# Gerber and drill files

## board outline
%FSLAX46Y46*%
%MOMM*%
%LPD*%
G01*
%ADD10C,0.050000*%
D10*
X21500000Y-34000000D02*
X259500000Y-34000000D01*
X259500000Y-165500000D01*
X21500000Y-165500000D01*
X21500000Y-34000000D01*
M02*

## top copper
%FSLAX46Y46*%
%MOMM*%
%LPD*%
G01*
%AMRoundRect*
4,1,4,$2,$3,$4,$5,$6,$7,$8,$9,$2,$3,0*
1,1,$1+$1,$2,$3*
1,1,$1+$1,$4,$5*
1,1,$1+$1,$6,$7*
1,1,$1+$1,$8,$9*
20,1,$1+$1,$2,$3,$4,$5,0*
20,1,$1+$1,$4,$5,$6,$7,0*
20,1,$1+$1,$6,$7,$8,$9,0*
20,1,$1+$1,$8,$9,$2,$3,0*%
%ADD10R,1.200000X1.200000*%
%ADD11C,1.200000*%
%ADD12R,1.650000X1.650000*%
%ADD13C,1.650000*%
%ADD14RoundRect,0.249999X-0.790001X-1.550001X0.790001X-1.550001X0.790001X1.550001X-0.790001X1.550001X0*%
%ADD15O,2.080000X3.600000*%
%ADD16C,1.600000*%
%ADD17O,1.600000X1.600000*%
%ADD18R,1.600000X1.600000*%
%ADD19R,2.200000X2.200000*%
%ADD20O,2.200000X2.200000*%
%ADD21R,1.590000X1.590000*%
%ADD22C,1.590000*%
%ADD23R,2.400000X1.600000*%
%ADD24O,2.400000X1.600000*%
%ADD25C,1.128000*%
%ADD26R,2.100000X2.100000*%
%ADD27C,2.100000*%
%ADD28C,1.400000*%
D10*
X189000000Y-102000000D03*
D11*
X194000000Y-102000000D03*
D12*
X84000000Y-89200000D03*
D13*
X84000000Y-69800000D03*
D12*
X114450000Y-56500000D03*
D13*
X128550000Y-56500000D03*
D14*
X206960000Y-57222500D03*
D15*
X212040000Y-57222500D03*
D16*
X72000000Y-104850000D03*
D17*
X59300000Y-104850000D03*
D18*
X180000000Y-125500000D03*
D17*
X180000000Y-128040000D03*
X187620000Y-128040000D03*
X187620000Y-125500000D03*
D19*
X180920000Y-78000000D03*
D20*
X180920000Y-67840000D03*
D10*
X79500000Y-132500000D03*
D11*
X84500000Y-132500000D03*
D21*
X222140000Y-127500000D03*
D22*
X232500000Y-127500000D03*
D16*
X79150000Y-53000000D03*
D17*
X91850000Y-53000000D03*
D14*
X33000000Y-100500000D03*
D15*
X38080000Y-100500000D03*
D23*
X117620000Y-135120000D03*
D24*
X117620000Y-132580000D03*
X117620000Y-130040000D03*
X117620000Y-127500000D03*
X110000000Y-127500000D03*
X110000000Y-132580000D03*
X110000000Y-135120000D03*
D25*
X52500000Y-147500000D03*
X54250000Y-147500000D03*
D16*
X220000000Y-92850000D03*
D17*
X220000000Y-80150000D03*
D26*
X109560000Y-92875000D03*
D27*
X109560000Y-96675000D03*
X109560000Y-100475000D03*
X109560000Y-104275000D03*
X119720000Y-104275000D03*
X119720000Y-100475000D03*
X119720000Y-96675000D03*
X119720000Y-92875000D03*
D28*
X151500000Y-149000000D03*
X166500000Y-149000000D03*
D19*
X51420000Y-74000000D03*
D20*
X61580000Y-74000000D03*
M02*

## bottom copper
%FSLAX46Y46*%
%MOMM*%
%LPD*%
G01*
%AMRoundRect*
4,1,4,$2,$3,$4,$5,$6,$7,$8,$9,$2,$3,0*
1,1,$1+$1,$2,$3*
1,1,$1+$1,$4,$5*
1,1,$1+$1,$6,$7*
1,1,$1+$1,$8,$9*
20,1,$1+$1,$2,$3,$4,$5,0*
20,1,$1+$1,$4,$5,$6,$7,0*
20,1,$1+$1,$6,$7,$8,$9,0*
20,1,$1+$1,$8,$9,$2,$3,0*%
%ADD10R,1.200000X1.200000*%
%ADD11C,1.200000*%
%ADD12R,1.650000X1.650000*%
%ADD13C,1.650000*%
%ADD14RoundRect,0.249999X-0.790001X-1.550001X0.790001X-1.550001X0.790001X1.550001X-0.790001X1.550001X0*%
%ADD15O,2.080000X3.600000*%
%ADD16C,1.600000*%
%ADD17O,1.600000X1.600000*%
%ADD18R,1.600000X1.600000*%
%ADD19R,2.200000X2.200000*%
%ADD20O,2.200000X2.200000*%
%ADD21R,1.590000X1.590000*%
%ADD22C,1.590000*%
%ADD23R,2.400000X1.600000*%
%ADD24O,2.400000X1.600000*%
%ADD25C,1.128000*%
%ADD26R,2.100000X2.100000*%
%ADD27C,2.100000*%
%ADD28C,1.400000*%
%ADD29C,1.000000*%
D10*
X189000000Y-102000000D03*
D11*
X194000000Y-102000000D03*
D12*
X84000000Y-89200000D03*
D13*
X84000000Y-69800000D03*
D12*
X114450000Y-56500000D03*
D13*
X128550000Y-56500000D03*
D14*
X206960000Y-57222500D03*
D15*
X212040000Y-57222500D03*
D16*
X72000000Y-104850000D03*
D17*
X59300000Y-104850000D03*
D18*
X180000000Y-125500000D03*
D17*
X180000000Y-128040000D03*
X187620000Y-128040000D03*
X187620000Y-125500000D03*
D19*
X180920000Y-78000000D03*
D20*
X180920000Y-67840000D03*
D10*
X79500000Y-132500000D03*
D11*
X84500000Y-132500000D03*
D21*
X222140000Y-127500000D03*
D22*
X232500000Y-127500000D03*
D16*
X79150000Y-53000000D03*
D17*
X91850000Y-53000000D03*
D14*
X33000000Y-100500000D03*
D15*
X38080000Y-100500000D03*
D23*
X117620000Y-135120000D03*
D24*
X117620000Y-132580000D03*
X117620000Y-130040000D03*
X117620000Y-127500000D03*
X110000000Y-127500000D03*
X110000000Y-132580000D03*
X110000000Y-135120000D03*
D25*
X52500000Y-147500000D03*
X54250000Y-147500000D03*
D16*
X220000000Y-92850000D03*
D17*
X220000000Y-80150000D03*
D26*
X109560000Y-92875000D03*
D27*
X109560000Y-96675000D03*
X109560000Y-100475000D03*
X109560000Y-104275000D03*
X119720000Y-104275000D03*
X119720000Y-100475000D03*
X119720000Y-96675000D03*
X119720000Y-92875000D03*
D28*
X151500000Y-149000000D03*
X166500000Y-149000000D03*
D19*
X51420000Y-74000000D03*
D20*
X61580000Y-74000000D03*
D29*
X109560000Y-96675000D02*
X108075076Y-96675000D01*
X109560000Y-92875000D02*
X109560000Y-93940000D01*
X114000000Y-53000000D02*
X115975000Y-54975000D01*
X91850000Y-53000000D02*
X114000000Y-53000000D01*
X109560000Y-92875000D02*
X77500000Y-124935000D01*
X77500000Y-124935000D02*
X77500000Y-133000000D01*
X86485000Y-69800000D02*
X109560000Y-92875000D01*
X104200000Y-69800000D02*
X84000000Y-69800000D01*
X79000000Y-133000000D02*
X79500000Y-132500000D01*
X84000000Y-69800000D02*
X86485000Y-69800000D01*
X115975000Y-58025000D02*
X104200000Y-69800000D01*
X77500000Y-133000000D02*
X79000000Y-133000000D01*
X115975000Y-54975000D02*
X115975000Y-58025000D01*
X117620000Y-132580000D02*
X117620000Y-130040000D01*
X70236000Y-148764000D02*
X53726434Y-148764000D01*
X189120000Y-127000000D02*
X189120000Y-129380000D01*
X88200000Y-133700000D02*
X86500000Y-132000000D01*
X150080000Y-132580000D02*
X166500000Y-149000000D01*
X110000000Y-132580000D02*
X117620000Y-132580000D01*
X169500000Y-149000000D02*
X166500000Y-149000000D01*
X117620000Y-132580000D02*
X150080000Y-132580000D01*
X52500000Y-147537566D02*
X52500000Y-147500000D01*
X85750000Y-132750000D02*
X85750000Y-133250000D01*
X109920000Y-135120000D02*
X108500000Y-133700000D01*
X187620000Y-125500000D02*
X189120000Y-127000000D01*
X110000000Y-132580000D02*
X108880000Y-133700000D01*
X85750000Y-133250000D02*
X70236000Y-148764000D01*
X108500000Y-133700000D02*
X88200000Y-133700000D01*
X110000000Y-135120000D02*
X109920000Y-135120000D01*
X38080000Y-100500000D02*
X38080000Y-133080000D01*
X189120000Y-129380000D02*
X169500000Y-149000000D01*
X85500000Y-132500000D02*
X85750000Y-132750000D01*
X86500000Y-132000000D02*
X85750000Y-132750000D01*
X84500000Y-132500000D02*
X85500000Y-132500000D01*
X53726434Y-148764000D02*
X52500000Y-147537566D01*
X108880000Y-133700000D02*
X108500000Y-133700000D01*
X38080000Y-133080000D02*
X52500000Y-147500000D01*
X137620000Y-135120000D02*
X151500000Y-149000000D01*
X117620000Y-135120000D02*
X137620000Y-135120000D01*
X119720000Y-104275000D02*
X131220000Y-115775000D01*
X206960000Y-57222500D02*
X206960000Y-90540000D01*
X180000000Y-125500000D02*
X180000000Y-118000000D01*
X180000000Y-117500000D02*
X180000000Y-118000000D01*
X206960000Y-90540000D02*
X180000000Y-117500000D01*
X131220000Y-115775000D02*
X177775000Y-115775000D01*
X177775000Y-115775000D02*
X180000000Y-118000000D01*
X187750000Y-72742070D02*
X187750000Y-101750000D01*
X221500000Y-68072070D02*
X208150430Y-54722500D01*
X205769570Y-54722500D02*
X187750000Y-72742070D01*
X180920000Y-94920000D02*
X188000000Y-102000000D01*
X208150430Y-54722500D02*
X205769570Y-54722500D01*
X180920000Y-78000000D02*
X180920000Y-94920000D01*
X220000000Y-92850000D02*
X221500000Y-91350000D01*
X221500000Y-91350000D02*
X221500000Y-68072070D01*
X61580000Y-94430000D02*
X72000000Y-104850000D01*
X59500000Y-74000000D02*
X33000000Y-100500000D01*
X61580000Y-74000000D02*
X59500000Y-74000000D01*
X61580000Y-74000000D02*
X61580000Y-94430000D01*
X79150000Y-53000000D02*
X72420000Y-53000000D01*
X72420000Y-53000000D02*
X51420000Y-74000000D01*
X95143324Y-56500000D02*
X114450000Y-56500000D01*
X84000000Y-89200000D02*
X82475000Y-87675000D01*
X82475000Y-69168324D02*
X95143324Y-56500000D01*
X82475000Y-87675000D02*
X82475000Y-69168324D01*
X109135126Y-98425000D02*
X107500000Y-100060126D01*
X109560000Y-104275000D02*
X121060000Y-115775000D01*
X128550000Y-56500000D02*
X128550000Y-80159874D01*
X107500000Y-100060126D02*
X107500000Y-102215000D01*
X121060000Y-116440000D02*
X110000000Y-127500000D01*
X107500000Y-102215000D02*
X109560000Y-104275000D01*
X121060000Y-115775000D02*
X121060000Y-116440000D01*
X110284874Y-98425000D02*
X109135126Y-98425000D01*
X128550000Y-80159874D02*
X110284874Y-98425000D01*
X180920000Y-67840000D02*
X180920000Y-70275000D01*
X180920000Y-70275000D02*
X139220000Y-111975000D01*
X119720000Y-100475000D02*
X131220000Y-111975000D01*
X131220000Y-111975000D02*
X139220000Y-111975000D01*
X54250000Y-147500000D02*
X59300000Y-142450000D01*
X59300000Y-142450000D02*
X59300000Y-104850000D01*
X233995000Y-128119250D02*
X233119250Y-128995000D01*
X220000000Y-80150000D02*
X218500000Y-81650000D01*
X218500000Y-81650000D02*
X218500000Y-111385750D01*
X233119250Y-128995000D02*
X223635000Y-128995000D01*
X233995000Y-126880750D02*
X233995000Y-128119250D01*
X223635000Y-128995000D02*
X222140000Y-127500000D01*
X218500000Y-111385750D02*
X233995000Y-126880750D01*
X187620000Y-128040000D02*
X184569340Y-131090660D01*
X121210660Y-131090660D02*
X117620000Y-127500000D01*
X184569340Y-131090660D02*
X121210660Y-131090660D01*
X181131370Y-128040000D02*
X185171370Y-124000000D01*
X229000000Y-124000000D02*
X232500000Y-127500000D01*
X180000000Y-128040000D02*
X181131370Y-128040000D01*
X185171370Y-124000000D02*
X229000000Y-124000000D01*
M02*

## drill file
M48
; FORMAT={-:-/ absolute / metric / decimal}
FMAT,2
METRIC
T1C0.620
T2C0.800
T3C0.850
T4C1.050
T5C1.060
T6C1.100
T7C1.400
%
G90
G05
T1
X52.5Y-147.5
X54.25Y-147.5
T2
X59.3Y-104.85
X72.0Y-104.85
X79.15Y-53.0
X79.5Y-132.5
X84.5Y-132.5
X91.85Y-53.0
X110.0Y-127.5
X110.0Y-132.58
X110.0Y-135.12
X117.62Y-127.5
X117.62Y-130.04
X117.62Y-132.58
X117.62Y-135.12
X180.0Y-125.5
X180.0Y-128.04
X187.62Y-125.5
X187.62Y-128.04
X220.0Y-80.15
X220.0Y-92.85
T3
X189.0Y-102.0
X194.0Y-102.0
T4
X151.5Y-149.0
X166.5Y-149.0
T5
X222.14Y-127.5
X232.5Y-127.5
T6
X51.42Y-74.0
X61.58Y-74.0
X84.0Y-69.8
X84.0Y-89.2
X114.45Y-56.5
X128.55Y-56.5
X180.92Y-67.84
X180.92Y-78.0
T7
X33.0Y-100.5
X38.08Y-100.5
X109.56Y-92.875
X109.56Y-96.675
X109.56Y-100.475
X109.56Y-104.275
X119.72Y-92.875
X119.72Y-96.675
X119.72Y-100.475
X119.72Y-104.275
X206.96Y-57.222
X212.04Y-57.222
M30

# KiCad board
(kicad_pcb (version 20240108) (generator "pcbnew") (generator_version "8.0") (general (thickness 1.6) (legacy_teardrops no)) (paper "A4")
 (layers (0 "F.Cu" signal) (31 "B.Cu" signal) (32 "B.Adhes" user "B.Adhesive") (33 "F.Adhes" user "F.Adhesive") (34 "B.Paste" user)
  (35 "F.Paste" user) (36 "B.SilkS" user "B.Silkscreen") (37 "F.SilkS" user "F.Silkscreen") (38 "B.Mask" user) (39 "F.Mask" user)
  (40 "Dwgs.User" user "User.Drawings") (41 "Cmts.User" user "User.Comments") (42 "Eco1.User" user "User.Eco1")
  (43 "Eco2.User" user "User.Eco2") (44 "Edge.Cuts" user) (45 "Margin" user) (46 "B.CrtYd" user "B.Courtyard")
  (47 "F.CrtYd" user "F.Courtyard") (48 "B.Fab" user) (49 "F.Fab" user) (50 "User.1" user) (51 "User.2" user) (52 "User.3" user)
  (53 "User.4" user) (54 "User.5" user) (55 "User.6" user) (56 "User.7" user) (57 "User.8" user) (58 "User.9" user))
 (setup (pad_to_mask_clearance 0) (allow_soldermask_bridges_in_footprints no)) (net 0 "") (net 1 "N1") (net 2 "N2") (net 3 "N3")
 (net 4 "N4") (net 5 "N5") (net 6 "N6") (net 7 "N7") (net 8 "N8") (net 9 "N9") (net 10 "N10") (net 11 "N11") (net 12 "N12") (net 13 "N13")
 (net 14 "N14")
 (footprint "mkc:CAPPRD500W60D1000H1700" (layer "F.Cu") (at 191.5 102)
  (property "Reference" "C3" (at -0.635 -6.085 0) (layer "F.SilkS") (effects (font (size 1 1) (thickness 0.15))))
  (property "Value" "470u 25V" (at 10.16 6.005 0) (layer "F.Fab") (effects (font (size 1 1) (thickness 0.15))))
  (pad "1" thru_hole rect (at -2.5 0) (size 1.2 1.2) (drill 0.85) (layers "*.Cu" "*.Mask") (remove_unused_layers no) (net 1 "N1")
   (solder_mask_margin 0.102))
  (pad "2" thru_hole circle (at 2.5 0) (size 1.2 1.2) (drill 0.85) (layers "*.Cu" "*.Mask") (remove_unused_layers no) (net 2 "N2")
   (solder_mask_margin 0.102)))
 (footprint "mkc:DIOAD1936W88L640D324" (layer "F.Cu") (at 84 89.2 90)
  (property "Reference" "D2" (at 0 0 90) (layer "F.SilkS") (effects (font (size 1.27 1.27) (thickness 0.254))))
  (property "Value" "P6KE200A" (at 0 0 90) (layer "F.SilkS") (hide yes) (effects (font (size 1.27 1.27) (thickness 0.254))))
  (pad "1" thru_hole rect (at 0 0 90) (size 1.65 1.65) (drill 1.1) (layers "*.Cu" "*.Mask") (remove_unused_layers no) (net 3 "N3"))
  (pad "2" thru_hole circle (at 19.4 0 90) (size 1.65 1.65) (drill 1.1) (layers "*.Cu" "*.Mask") (remove_unused_layers no) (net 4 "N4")))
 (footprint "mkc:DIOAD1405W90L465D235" (layer "F.Cu") (at 114.45 56.5)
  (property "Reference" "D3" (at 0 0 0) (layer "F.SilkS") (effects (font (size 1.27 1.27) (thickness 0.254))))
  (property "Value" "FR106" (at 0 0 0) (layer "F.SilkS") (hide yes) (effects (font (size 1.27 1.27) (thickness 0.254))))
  (pad "1" thru_hole rect (at 0 0) (size 1.65 1.65) (drill 1.1) (layers "*.Cu" "*.Mask") (remove_unused_layers no) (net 3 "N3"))
  (pad "2" thru_hole circle (at 14.1 0) (size 1.65 1.65) (drill 1.1) (layers "*.Cu" "*.Mask") (remove_unused_layers no) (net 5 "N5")))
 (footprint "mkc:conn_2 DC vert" (layer "F.Cu") (at 206.96 57.2225)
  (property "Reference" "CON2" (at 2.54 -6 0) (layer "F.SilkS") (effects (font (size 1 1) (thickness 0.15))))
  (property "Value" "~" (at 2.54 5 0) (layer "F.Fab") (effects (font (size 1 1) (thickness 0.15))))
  (pad "1" thru_hole roundrect (at 0 0) (size 2.08 3.6) (drill 1.4) (layers "*.Cu" "*.Mask") (remove_unused_layers no)
   (roundrect_rratio 0.120192) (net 2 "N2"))
  (pad "2" thru_hole oval (at 5.08 0) (size 2.08 3.6) (drill 1.4) (layers "*.Cu" "*.Mask") (remove_unused_layers no) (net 1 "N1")))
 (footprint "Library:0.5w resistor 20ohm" (layer "F.Cu") (at 72 104.85 180)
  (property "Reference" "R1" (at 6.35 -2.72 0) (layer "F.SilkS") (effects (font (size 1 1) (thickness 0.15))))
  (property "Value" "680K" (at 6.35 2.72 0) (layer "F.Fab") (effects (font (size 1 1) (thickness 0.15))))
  (pad "1" thru_hole circle (at 0 0 180) (size 1.6 1.6) (drill 0.8) (layers "*.Cu" "*.Mask") (remove_unused_layers no) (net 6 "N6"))
  (pad "2" thru_hole oval (at 12.7 0 180) (size 1.6 1.6) (drill 0.8) (layers "*.Cu" "*.Mask") (remove_unused_layers no) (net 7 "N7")))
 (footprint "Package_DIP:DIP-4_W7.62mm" (layer "F.Cu") (at 180 125.5)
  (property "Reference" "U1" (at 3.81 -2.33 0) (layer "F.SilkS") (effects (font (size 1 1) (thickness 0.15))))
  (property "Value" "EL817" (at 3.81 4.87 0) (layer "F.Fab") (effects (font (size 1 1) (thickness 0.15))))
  (pad "1" thru_hole rect (at 0 0) (size 1.6 1.6) (drill 0.8) (layers "*.Cu" "*.Mask") (remove_unused_layers no) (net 2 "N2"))
  (pad "2" thru_hole oval (at 0 2.54) (size 1.6 1.6) (drill 0.8) (layers "*.Cu" "*.Mask") (remove_unused_layers no) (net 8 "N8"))
  (pad "3" thru_hole oval (at 7.62 2.54) (size 1.6 1.6) (drill 0.8) (layers "*.Cu" "*.Mask") (remove_unused_layers no) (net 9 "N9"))
  (pad "4" thru_hole oval (at 7.62 0) (size 1.6 1.6) (drill 0.8) (layers "*.Cu" "*.Mask") (remove_unused_layers no) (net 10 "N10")))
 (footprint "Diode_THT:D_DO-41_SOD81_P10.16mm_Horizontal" (layer "F.Cu") (at 180.92 78 90)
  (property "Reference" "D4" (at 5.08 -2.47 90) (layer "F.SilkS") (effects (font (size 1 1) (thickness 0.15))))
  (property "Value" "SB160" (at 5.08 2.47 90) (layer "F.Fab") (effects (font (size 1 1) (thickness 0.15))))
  (pad "1" thru_hole rect (at 0 0 90) (size 2.2 2.2) (drill 1.1) (layers "*.Cu" "*.Mask") (remove_unused_layers no) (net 1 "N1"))
  (pad "2" thru_hole oval (at 10.16 0 90) (size 2.2 2.2) (drill 1.1) (layers "*.Cu" "*.Mask") (remove_unused_layers no) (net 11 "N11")))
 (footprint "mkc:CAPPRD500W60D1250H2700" (layer "F.Cu") (at 82 132.5)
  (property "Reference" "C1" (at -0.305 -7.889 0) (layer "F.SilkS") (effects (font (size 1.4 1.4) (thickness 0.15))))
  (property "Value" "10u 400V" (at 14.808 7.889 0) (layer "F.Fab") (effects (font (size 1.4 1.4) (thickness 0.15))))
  (pad "1" thru_hole rect (at -2.5 0) (size 1.2 1.2) (drill 0.8) (layers "*.Cu" "*.Mask") (remove_unused_layers no) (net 4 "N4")
   (solder_mask_margin 0.102))
  (pad "2" thru_hole circle (at 2.5 0) (size 1.2 1.2) (drill 0.8) (layers "*.Cu" "*.Mask") (remove_unused_layers no) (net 10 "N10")
   (solder_mask_margin 0.102)))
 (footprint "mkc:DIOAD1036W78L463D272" (layer "F.Cu") (at 227.32 127.5)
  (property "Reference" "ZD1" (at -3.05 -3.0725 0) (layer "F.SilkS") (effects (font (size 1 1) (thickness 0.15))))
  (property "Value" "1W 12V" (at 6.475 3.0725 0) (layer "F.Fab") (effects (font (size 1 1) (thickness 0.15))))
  (pad "1" thru_hole rect (at -5.18 0) (size 1.59 1.59) (drill 1.06) (layers "*.Cu" "*.Mask") (remove_unused_layers no) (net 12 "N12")
   (solder_mask_margin 0.102))
  (pad "2" thru_hole circle (at 5.18 0) (size 1.59 1.59) (drill 1.06) (layers "*.Cu" "*.Mask") (remove_unused_layers no) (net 8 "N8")
   (solder_mask_margin 0.102)))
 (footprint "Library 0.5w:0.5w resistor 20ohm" (layer "F.Cu") (at 79.15 53)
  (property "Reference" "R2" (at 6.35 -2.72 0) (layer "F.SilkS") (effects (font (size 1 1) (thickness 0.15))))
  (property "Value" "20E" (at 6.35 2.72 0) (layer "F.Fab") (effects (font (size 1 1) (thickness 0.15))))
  (pad "1" thru_hole circle (at 0 0) (size 1.6 1.6) (drill 0.8) (layers "*.Cu" "*.Mask") (remove_unused_layers no) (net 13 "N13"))
  (pad "2" thru_hole oval (at 12.7 0) (size 1.6 1.6) (drill 0.8) (layers "*.Cu" "*.Mask") (remove_unused_layers no) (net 4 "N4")))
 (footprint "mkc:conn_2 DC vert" (layer "F.Cu") (at 33 100.5)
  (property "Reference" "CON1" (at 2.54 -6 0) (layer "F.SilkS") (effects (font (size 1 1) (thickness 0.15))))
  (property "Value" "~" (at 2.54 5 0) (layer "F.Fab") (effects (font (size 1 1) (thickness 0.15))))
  (pad "1" thru_hole roundrect (at 0 0) (size 2.08 3.6) (drill 1.4) (layers "*.Cu" "*.Mask") (remove_unused_layers no)
   (roundrect_rratio 0.120192) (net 6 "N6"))
  (pad "2" thru_hole oval (at 5.08 0) (size 2.08 3.6) (drill 1.4) (layers "*.Cu" "*.Mask") (remove_unused_layers no) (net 10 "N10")))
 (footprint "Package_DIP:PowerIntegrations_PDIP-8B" (layer "F.Cu") (at 117.62 135.12 180)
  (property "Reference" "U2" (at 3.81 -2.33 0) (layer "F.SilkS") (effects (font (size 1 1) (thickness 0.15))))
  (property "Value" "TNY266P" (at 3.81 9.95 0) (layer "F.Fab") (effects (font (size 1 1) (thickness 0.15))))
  (pad "1" thru_hole rect (at 0 0 180) (size 2.4 1.6) (drill 0.8) (layers "*.Cu" "*.Mask") (remove_unused_layers no) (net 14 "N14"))
  (pad "2" thru_hole oval (at 0 2.54 180) (size 2.4 1.6) (drill 0.8) (layers "*.Cu" "*.Mask") (remove_unused_layers no) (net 10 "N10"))
  (pad "3" thru_hole oval (at 0 5.08 180) (size 2.4 1.6) (drill 0.8) (layers "*.Cu" "*.Mask") (remove_unused_layers no) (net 10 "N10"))
  (pad "4" thru_hole oval (at 0 7.62 180) (size 2.4 1.6) (drill 0.8) (layers "*.Cu" "*.Mask") (remove_unused_layers no) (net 9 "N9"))
  (pad "5" thru_hole oval (at 7.62 7.62 180) (size 2.4 1.6) (drill 0.8) (layers "*.Cu" "*.Mask") (remove_unused_layers no) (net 5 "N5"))
  (pad "7" thru_hole oval (at 7.62 2.54 180) (size 2.4 1.6) (drill 0.8) (layers "*.Cu" "*.Mask") (remove_unused_layers no) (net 10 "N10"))
  (pad "8" thru_hole oval (at 7.62 0 180) (size 2.4 1.6) (drill 0.8) (layers "*.Cu" "*.Mask") (remove_unused_layers no) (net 10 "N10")))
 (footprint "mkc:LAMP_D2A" (layer "F.Cu") (at 53.375 147.5)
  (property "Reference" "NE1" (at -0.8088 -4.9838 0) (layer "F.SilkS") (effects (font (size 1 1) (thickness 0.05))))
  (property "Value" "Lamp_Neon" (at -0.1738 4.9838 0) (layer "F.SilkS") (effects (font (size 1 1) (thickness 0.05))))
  (pad "1" thru_hole circle (at -0.875 0) (size 1.128 1.128) (drill 0.62) (layers "*.Cu" "*.Mask") (remove_unused_layers no) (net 10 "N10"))
  (pad "2" thru_hole circle (at 0.875 0) (size 1.128 1.128) (drill 0.62) (layers "*.Cu" "*.Mask") (remove_unused_layers no) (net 7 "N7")))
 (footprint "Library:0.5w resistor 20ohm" (layer "F.Cu") (at 220 92.85 90)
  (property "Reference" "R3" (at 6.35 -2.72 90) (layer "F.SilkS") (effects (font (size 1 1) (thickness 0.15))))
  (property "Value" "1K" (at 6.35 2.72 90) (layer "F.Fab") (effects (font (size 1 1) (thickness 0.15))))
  (pad "1" thru_hole circle (at 0 0 90) (size 1.6 1.6) (drill 0.8) (layers "*.Cu" "*.Mask") (remove_unused_layers no) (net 1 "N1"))
  (pad "2" thru_hole oval (at 12.7 0 90) (size 1.6 1.6) (drill 0.8) (layers "*.Cu" "*.Mask") (remove_unused_layers no) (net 12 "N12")))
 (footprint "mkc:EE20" (layer "F.Cu") (at 109.56 92.875)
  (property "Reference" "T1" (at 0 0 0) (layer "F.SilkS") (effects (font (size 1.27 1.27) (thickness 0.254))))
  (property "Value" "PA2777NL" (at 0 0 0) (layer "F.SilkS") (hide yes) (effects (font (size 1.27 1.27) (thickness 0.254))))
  (pad "1" thru_hole rect (at 0 0) (size 2.1 2.1) (drill 1.4) (layers "*.Cu" "*.Mask") (remove_unused_layers no) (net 4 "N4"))
  (pad "2" thru_hole circle (at 0 3.8) (size 2.1 2.1) (drill 1.4) (layers "*.Cu" "*.Mask") (remove_unused_layers no))
  (pad "3" thru_hole circle (at 0 7.6) (size 2.1 2.1) (drill 1.4) (layers "*.Cu" "*.Mask") (remove_unused_layers no))
  (pad "4" thru_hole circle (at 0 11.4) (size 2.1 2.1) (drill 1.4) (layers "*.Cu" "*.Mask") (remove_unused_layers no) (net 5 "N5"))
  (pad "7" thru_hole circle (at 10.16 11.4) (size 2.1 2.1) (drill 1.4) (layers "*.Cu" "*.Mask") (remove_unused_layers no) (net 2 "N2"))
  (pad "8" thru_hole circle (at 10.16 7.6) (size 2.1 2.1) (drill 1.4) (layers "*.Cu" "*.Mask") (remove_unused_layers no) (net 11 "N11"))
  (pad "9" thru_hole circle (at 10.16 3.8) (size 2.1 2.1) (drill 1.4) (layers "*.Cu" "*.Mask") (remove_unused_layers no))
  (pad "10" thru_hole circle (at 10.16 0) (size 2.1 2.1) (drill 1.4) (layers "*.Cu" "*.Mask") (remove_unused_layers no)))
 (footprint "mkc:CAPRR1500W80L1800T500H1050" (layer "F.Cu") (at 159 149)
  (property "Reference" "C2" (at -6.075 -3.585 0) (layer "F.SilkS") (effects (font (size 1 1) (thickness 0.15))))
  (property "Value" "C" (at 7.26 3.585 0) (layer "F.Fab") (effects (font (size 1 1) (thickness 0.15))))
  (pad "1" thru_hole circle (at -7.5 0) (size 1.4 1.4) (drill 1.05) (layers "*.Cu" "*.Mask") (remove_unused_layers no) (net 14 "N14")
   (solder_mask_margin 0.102))
  (pad "2" thru_hole circle (at 7.5 0) (size 1.4 1.4) (drill 1.05) (layers "*.Cu" "*.Mask") (remove_unused_layers no) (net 10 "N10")
   (solder_mask_margin 0.102)))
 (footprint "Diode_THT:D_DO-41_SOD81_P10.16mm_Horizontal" (layer "F.Cu") (at 51.42 74)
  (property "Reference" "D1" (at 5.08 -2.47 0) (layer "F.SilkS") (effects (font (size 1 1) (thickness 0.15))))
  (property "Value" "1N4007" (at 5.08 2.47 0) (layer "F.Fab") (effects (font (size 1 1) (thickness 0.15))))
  (pad "1" thru_hole rect (at 0 0) (size 2.2 2.2) (drill 1.1) (layers "*.Cu" "*.Mask") (remove_unused_layers no) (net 13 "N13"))
  (pad "2" thru_hole oval (at 10.16 0) (size 2.2 2.2) (drill 1.1) (layers "*.Cu" "*.Mask") (remove_unused_layers no) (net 6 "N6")))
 (gr_rect (start 21.5 34) (end 259.5 165.5) (stroke (width 0.05) (type default)) (fill none) (layer "Edge.Cuts"))
 (segment (start 109.56 96.675) (end 108.075076 96.675) (width 1) (layer "B.Cu") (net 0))
 (segment (start 109.56 92.875) (end 109.56 93.94) (width 1) (layer "B.Cu") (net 4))
 (segment (start 114 53) (end 115.975 54.975) (width 1) (layer "B.Cu") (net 4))
 (segment (start 91.85 53) (end 114 53) (width 1) (layer "B.Cu") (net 4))
 (segment (start 109.56 92.875) (end 77.5 124.935) (width 1) (layer "B.Cu") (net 4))
 (segment (start 77.5 124.935) (end 77.5 133) (width 1) (layer "B.Cu") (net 4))
 (segment (start 86.485 69.8) (end 109.56 92.875) (width 1) (layer "B.Cu") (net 4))
 (segment (start 104.2 69.8) (end 84 69.8) (width 1) (layer "B.Cu") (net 4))
 (segment (start 79 133) (end 79.5 132.5) (width 1) (layer "B.Cu") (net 4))
 (segment (start 84 69.8) (end 86.485 69.8) (width 1) (layer "B.Cu") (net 4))
 (segment (start 115.975 58.025) (end 104.2 69.8) (width 1) (layer "B.Cu") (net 4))
 (segment (start 77.5 133) (end 79 133) (width 1) (layer "B.Cu") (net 4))
 (segment (start 115.975 54.975) (end 115.975 58.025) (width 1) (layer "B.Cu") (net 4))
 (segment (start 117.62 132.58) (end 117.62 130.04) (width 1) (layer "B.Cu") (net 10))
 (segment (start 70.236 148.764) (end 53.726434 148.764) (width 1) (layer "B.Cu") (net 10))
 (segment (start 189.12 127) (end 189.12 129.38) (width 1) (layer "B.Cu") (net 10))
 (segment (start 88.2 133.7) (end 86.5 132) (width 1) (layer "B.Cu") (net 10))
 (segment (start 150.08 132.58) (end 166.5 149) (width 1) (layer "B.Cu") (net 10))
 (segment (start 110 132.58) (end 117.62 132.58) (width 1) (layer "B.Cu") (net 10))
 (segment (start 169.5 149) (end 166.5 149) (width 1) (layer "B.Cu") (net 10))
 (segment (start 117.62 132.58) (end 150.08 132.58) (width 1) (layer "B.Cu") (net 10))
 (segment (start 52.5 147.537566) (end 52.5 147.5) (width 1) (layer "B.Cu") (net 10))
 (segment (start 85.75 132.75) (end 85.75 133.25) (width 1) (layer "B.Cu") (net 10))
 (segment (start 109.92 135.12) (end 108.5 133.7) (width 1) (layer "B.Cu") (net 10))
 (segment (start 187.62 125.5) (end 189.12 127) (width 1) (layer "B.Cu") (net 10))
 (segment (start 110 132.58) (end 108.88 133.7) (width 1) (layer "B.Cu") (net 10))
 (segment (start 85.75 133.25) (end 70.236 148.764) (width 1) (layer "B.Cu") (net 10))
 (segment (start 108.5 133.7) (end 88.2 133.7) (width 1) (layer "B.Cu") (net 10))
 (segment (start 110 135.12) (end 109.92 135.12) (width 1) (layer "B.Cu") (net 10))
 (segment (start 38.08 100.5) (end 38.08 133.08) (width 1) (layer "B.Cu") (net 10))
 (segment (start 189.12 129.38) (end 169.5 149) (width 1) (layer "B.Cu") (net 10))
 (segment (start 85.5 132.5) (end 85.75 132.75) (width 1) (layer "B.Cu") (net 10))
 (segment (start 86.5 132) (end 85.75 132.75) (width 1) (layer "B.Cu") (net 10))
 (segment (start 84.5 132.5) (end 85.5 132.5) (width 1) (layer "B.Cu") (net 10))
 (segment (start 53.726434 148.764) (end 52.5 147.537566) (width 1) (layer "B.Cu") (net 10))
 (segment (start 108.88 133.7) (end 108.5 133.7) (width 1) (layer "B.Cu") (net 10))
 (segment (start 38.08 133.08) (end 52.5 147.5) (width 1) (layer "B.Cu") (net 10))
 (segment (start 137.62 135.12) (end 151.5 149) (width 1) (layer "B.Cu") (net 14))
 (segment (start 117.62 135.12) (end 137.62 135.12) (width 1) (layer "B.Cu") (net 14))
 (segment (start 119.72 104.275) (end 131.22 115.775) (width 1) (layer "B.Cu") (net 2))
 (segment (start 206.96 57.2225) (end 206.96 90.54) (width 1) (layer "B.Cu") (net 2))
 (segment (start 180 125.5) (end 180 118) (width 1) (layer "B.Cu") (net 2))
 (segment (start 180 117.5) (end 180 118) (width 1) (layer "B.Cu") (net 2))
 (segment (start 206.96 90.54) (end 180 117.5) (width 1) (layer "B.Cu") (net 2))
 (segment (start 131.22 115.775) (end 177.775 115.775) (width 1) (layer "B.Cu") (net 2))
 (segment (start 177.775 115.775) (end 180 118) (width 1) (layer "B.Cu") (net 2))
 (segment (start 187.75 72.74207) (end 187.75 101.75) (width 1) (layer "B.Cu") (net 1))
 (segment (start 221.5 68.07207) (end 208.15043 54.7225) (width 1) (layer "B.Cu") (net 1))
 (segment (start 205.76957 54.7225) (end 187.75 72.74207) (width 1) (layer "B.Cu") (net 1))
 (segment (start 180.92 94.92) (end 188 102) (width 1) (layer "B.Cu") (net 1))
 (segment (start 208.15043 54.7225) (end 205.76957 54.7225) (width 1) (layer "B.Cu") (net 1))
 (segment (start 180.92 78) (end 180.92 94.92) (width 1) (layer "B.Cu") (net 1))
 (segment (start 220 92.85) (end 221.5 91.35) (width 1) (layer "B.Cu") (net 1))
 (segment (start 221.5 91.35) (end 221.5 68.07207) (width 1) (layer "B.Cu") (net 1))
 (segment (start 61.58 94.43) (end 72 104.85) (width 1) (layer "B.Cu") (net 6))
 (segment (start 59.5 74) (end 33 100.5) (width 1) (layer "B.Cu") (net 6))
 (segment (start 61.58 74) (end 59.5 74) (width 1) (layer "B.Cu") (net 6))
 (segment (start 61.58 74) (end 61.58 94.43) (width 1) (layer "B.Cu") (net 6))
 (segment (start 79.15 53) (end 72.42 53) (width 1) (layer "B.Cu") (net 13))
 (segment (start 72.42 53) (end 51.42 74) (width 1) (layer "B.Cu") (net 13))
 (segment (start 95.143324 56.5) (end 114.45 56.5) (width 1) (layer "B.Cu") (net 3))
 (segment (start 84 89.2) (end 82.475 87.675) (width 1) (layer "B.Cu") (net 3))
 (segment (start 82.475 69.168324) (end 95.143324 56.5) (width 1) (layer "B.Cu") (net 3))
 (segment (start 82.475 87.675) (end 82.475 69.168324) (width 1) (layer "B.Cu") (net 3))
 (segment (start 109.135126 98.425) (end 107.5 100.060126) (width 1) (layer "B.Cu") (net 5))
 (segment (start 109.56 104.275) (end 121.06 115.775) (width 1) (layer "B.Cu") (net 5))
 (segment (start 128.55 56.5) (end 128.55 80.159874) (width 1) (layer "B.Cu") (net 5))
 (segment (start 107.5 100.060126) (end 107.5 102.215) (width 1) (layer "B.Cu") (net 5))
 (segment (start 121.06 116.44) (end 110 127.5) (width 1) (layer "B.Cu") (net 5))
 (segment (start 107.5 102.215) (end 109.56 104.275) (width 1) (layer "B.Cu") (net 5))
 (segment (start 121.06 115.775) (end 121.06 116.44) (width 1) (layer "B.Cu") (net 5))
 (segment (start 110.284874 98.425) (end 109.135126 98.425) (width 1) (layer "B.Cu") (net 5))
 (segment (start 128.55 80.159874) (end 110.284874 98.425) (width 1) (layer "B.Cu") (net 5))
 (segment (start 180.92 67.84) (end 180.92 70.275) (width 1) (layer "B.Cu") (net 11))
 (segment (start 180.92 70.275) (end 139.22 111.975) (width 1) (layer "B.Cu") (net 11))
 (segment (start 119.72 100.475) (end 131.22 111.975) (width 1) (layer "B.Cu") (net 11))
 (segment (start 131.22 111.975) (end 139.22 111.975) (width 1) (layer "B.Cu") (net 11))
 (segment (start 54.25 147.5) (end 59.3 142.45) (width 1) (layer "B.Cu") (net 7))
 (segment (start 59.3 142.45) (end 59.3 104.85) (width 1) (layer "B.Cu") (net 7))
 (segment (start 233.995 128.11925) (end 233.11925 128.995) (width 1) (layer "B.Cu") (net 12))
 (segment (start 220 80.15) (end 218.5 81.65) (width 1) (layer "B.Cu") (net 12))
 (segment (start 218.5 81.65) (end 218.5 111.38575) (width 1) (layer "B.Cu") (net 12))
 (segment (start 233.11925 128.995) (end 223.635 128.995) (width 1) (layer "B.Cu") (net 12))
 (segment (start 233.995 126.88075) (end 233.995 128.11925) (width 1) (layer "B.Cu") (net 12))
 (segment (start 223.635 128.995) (end 222.14 127.5) (width 1) (layer "B.Cu") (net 12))
 (segment (start 218.5 111.38575) (end 233.995 126.88075) (width 1) (layer "B.Cu") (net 12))
 (segment (start 187.62 128.04) (end 184.56934 131.09066) (width 1) (layer "B.Cu") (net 9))
 (segment (start 121.21066 131.09066) (end 117.62 127.5) (width 1) (layer "B.Cu") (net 9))
 (segment (start 184.56934 131.09066) (end 121.21066 131.09066) (width 1) (layer "B.Cu") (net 9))
 (segment (start 181.13137 128.04) (end 185.17137 124) (width 1) (layer "B.Cu") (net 8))
 (segment (start 229 124) (end 232.5 127.5) (width 1) (layer "B.Cu") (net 8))
 (segment (start 180 128.04) (end 181.13137 128.04) (width 1) (layer "B.Cu") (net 8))
 (segment (start 185.17137 124) (end 229 124) (width 1) (layer "B.Cu") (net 8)))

